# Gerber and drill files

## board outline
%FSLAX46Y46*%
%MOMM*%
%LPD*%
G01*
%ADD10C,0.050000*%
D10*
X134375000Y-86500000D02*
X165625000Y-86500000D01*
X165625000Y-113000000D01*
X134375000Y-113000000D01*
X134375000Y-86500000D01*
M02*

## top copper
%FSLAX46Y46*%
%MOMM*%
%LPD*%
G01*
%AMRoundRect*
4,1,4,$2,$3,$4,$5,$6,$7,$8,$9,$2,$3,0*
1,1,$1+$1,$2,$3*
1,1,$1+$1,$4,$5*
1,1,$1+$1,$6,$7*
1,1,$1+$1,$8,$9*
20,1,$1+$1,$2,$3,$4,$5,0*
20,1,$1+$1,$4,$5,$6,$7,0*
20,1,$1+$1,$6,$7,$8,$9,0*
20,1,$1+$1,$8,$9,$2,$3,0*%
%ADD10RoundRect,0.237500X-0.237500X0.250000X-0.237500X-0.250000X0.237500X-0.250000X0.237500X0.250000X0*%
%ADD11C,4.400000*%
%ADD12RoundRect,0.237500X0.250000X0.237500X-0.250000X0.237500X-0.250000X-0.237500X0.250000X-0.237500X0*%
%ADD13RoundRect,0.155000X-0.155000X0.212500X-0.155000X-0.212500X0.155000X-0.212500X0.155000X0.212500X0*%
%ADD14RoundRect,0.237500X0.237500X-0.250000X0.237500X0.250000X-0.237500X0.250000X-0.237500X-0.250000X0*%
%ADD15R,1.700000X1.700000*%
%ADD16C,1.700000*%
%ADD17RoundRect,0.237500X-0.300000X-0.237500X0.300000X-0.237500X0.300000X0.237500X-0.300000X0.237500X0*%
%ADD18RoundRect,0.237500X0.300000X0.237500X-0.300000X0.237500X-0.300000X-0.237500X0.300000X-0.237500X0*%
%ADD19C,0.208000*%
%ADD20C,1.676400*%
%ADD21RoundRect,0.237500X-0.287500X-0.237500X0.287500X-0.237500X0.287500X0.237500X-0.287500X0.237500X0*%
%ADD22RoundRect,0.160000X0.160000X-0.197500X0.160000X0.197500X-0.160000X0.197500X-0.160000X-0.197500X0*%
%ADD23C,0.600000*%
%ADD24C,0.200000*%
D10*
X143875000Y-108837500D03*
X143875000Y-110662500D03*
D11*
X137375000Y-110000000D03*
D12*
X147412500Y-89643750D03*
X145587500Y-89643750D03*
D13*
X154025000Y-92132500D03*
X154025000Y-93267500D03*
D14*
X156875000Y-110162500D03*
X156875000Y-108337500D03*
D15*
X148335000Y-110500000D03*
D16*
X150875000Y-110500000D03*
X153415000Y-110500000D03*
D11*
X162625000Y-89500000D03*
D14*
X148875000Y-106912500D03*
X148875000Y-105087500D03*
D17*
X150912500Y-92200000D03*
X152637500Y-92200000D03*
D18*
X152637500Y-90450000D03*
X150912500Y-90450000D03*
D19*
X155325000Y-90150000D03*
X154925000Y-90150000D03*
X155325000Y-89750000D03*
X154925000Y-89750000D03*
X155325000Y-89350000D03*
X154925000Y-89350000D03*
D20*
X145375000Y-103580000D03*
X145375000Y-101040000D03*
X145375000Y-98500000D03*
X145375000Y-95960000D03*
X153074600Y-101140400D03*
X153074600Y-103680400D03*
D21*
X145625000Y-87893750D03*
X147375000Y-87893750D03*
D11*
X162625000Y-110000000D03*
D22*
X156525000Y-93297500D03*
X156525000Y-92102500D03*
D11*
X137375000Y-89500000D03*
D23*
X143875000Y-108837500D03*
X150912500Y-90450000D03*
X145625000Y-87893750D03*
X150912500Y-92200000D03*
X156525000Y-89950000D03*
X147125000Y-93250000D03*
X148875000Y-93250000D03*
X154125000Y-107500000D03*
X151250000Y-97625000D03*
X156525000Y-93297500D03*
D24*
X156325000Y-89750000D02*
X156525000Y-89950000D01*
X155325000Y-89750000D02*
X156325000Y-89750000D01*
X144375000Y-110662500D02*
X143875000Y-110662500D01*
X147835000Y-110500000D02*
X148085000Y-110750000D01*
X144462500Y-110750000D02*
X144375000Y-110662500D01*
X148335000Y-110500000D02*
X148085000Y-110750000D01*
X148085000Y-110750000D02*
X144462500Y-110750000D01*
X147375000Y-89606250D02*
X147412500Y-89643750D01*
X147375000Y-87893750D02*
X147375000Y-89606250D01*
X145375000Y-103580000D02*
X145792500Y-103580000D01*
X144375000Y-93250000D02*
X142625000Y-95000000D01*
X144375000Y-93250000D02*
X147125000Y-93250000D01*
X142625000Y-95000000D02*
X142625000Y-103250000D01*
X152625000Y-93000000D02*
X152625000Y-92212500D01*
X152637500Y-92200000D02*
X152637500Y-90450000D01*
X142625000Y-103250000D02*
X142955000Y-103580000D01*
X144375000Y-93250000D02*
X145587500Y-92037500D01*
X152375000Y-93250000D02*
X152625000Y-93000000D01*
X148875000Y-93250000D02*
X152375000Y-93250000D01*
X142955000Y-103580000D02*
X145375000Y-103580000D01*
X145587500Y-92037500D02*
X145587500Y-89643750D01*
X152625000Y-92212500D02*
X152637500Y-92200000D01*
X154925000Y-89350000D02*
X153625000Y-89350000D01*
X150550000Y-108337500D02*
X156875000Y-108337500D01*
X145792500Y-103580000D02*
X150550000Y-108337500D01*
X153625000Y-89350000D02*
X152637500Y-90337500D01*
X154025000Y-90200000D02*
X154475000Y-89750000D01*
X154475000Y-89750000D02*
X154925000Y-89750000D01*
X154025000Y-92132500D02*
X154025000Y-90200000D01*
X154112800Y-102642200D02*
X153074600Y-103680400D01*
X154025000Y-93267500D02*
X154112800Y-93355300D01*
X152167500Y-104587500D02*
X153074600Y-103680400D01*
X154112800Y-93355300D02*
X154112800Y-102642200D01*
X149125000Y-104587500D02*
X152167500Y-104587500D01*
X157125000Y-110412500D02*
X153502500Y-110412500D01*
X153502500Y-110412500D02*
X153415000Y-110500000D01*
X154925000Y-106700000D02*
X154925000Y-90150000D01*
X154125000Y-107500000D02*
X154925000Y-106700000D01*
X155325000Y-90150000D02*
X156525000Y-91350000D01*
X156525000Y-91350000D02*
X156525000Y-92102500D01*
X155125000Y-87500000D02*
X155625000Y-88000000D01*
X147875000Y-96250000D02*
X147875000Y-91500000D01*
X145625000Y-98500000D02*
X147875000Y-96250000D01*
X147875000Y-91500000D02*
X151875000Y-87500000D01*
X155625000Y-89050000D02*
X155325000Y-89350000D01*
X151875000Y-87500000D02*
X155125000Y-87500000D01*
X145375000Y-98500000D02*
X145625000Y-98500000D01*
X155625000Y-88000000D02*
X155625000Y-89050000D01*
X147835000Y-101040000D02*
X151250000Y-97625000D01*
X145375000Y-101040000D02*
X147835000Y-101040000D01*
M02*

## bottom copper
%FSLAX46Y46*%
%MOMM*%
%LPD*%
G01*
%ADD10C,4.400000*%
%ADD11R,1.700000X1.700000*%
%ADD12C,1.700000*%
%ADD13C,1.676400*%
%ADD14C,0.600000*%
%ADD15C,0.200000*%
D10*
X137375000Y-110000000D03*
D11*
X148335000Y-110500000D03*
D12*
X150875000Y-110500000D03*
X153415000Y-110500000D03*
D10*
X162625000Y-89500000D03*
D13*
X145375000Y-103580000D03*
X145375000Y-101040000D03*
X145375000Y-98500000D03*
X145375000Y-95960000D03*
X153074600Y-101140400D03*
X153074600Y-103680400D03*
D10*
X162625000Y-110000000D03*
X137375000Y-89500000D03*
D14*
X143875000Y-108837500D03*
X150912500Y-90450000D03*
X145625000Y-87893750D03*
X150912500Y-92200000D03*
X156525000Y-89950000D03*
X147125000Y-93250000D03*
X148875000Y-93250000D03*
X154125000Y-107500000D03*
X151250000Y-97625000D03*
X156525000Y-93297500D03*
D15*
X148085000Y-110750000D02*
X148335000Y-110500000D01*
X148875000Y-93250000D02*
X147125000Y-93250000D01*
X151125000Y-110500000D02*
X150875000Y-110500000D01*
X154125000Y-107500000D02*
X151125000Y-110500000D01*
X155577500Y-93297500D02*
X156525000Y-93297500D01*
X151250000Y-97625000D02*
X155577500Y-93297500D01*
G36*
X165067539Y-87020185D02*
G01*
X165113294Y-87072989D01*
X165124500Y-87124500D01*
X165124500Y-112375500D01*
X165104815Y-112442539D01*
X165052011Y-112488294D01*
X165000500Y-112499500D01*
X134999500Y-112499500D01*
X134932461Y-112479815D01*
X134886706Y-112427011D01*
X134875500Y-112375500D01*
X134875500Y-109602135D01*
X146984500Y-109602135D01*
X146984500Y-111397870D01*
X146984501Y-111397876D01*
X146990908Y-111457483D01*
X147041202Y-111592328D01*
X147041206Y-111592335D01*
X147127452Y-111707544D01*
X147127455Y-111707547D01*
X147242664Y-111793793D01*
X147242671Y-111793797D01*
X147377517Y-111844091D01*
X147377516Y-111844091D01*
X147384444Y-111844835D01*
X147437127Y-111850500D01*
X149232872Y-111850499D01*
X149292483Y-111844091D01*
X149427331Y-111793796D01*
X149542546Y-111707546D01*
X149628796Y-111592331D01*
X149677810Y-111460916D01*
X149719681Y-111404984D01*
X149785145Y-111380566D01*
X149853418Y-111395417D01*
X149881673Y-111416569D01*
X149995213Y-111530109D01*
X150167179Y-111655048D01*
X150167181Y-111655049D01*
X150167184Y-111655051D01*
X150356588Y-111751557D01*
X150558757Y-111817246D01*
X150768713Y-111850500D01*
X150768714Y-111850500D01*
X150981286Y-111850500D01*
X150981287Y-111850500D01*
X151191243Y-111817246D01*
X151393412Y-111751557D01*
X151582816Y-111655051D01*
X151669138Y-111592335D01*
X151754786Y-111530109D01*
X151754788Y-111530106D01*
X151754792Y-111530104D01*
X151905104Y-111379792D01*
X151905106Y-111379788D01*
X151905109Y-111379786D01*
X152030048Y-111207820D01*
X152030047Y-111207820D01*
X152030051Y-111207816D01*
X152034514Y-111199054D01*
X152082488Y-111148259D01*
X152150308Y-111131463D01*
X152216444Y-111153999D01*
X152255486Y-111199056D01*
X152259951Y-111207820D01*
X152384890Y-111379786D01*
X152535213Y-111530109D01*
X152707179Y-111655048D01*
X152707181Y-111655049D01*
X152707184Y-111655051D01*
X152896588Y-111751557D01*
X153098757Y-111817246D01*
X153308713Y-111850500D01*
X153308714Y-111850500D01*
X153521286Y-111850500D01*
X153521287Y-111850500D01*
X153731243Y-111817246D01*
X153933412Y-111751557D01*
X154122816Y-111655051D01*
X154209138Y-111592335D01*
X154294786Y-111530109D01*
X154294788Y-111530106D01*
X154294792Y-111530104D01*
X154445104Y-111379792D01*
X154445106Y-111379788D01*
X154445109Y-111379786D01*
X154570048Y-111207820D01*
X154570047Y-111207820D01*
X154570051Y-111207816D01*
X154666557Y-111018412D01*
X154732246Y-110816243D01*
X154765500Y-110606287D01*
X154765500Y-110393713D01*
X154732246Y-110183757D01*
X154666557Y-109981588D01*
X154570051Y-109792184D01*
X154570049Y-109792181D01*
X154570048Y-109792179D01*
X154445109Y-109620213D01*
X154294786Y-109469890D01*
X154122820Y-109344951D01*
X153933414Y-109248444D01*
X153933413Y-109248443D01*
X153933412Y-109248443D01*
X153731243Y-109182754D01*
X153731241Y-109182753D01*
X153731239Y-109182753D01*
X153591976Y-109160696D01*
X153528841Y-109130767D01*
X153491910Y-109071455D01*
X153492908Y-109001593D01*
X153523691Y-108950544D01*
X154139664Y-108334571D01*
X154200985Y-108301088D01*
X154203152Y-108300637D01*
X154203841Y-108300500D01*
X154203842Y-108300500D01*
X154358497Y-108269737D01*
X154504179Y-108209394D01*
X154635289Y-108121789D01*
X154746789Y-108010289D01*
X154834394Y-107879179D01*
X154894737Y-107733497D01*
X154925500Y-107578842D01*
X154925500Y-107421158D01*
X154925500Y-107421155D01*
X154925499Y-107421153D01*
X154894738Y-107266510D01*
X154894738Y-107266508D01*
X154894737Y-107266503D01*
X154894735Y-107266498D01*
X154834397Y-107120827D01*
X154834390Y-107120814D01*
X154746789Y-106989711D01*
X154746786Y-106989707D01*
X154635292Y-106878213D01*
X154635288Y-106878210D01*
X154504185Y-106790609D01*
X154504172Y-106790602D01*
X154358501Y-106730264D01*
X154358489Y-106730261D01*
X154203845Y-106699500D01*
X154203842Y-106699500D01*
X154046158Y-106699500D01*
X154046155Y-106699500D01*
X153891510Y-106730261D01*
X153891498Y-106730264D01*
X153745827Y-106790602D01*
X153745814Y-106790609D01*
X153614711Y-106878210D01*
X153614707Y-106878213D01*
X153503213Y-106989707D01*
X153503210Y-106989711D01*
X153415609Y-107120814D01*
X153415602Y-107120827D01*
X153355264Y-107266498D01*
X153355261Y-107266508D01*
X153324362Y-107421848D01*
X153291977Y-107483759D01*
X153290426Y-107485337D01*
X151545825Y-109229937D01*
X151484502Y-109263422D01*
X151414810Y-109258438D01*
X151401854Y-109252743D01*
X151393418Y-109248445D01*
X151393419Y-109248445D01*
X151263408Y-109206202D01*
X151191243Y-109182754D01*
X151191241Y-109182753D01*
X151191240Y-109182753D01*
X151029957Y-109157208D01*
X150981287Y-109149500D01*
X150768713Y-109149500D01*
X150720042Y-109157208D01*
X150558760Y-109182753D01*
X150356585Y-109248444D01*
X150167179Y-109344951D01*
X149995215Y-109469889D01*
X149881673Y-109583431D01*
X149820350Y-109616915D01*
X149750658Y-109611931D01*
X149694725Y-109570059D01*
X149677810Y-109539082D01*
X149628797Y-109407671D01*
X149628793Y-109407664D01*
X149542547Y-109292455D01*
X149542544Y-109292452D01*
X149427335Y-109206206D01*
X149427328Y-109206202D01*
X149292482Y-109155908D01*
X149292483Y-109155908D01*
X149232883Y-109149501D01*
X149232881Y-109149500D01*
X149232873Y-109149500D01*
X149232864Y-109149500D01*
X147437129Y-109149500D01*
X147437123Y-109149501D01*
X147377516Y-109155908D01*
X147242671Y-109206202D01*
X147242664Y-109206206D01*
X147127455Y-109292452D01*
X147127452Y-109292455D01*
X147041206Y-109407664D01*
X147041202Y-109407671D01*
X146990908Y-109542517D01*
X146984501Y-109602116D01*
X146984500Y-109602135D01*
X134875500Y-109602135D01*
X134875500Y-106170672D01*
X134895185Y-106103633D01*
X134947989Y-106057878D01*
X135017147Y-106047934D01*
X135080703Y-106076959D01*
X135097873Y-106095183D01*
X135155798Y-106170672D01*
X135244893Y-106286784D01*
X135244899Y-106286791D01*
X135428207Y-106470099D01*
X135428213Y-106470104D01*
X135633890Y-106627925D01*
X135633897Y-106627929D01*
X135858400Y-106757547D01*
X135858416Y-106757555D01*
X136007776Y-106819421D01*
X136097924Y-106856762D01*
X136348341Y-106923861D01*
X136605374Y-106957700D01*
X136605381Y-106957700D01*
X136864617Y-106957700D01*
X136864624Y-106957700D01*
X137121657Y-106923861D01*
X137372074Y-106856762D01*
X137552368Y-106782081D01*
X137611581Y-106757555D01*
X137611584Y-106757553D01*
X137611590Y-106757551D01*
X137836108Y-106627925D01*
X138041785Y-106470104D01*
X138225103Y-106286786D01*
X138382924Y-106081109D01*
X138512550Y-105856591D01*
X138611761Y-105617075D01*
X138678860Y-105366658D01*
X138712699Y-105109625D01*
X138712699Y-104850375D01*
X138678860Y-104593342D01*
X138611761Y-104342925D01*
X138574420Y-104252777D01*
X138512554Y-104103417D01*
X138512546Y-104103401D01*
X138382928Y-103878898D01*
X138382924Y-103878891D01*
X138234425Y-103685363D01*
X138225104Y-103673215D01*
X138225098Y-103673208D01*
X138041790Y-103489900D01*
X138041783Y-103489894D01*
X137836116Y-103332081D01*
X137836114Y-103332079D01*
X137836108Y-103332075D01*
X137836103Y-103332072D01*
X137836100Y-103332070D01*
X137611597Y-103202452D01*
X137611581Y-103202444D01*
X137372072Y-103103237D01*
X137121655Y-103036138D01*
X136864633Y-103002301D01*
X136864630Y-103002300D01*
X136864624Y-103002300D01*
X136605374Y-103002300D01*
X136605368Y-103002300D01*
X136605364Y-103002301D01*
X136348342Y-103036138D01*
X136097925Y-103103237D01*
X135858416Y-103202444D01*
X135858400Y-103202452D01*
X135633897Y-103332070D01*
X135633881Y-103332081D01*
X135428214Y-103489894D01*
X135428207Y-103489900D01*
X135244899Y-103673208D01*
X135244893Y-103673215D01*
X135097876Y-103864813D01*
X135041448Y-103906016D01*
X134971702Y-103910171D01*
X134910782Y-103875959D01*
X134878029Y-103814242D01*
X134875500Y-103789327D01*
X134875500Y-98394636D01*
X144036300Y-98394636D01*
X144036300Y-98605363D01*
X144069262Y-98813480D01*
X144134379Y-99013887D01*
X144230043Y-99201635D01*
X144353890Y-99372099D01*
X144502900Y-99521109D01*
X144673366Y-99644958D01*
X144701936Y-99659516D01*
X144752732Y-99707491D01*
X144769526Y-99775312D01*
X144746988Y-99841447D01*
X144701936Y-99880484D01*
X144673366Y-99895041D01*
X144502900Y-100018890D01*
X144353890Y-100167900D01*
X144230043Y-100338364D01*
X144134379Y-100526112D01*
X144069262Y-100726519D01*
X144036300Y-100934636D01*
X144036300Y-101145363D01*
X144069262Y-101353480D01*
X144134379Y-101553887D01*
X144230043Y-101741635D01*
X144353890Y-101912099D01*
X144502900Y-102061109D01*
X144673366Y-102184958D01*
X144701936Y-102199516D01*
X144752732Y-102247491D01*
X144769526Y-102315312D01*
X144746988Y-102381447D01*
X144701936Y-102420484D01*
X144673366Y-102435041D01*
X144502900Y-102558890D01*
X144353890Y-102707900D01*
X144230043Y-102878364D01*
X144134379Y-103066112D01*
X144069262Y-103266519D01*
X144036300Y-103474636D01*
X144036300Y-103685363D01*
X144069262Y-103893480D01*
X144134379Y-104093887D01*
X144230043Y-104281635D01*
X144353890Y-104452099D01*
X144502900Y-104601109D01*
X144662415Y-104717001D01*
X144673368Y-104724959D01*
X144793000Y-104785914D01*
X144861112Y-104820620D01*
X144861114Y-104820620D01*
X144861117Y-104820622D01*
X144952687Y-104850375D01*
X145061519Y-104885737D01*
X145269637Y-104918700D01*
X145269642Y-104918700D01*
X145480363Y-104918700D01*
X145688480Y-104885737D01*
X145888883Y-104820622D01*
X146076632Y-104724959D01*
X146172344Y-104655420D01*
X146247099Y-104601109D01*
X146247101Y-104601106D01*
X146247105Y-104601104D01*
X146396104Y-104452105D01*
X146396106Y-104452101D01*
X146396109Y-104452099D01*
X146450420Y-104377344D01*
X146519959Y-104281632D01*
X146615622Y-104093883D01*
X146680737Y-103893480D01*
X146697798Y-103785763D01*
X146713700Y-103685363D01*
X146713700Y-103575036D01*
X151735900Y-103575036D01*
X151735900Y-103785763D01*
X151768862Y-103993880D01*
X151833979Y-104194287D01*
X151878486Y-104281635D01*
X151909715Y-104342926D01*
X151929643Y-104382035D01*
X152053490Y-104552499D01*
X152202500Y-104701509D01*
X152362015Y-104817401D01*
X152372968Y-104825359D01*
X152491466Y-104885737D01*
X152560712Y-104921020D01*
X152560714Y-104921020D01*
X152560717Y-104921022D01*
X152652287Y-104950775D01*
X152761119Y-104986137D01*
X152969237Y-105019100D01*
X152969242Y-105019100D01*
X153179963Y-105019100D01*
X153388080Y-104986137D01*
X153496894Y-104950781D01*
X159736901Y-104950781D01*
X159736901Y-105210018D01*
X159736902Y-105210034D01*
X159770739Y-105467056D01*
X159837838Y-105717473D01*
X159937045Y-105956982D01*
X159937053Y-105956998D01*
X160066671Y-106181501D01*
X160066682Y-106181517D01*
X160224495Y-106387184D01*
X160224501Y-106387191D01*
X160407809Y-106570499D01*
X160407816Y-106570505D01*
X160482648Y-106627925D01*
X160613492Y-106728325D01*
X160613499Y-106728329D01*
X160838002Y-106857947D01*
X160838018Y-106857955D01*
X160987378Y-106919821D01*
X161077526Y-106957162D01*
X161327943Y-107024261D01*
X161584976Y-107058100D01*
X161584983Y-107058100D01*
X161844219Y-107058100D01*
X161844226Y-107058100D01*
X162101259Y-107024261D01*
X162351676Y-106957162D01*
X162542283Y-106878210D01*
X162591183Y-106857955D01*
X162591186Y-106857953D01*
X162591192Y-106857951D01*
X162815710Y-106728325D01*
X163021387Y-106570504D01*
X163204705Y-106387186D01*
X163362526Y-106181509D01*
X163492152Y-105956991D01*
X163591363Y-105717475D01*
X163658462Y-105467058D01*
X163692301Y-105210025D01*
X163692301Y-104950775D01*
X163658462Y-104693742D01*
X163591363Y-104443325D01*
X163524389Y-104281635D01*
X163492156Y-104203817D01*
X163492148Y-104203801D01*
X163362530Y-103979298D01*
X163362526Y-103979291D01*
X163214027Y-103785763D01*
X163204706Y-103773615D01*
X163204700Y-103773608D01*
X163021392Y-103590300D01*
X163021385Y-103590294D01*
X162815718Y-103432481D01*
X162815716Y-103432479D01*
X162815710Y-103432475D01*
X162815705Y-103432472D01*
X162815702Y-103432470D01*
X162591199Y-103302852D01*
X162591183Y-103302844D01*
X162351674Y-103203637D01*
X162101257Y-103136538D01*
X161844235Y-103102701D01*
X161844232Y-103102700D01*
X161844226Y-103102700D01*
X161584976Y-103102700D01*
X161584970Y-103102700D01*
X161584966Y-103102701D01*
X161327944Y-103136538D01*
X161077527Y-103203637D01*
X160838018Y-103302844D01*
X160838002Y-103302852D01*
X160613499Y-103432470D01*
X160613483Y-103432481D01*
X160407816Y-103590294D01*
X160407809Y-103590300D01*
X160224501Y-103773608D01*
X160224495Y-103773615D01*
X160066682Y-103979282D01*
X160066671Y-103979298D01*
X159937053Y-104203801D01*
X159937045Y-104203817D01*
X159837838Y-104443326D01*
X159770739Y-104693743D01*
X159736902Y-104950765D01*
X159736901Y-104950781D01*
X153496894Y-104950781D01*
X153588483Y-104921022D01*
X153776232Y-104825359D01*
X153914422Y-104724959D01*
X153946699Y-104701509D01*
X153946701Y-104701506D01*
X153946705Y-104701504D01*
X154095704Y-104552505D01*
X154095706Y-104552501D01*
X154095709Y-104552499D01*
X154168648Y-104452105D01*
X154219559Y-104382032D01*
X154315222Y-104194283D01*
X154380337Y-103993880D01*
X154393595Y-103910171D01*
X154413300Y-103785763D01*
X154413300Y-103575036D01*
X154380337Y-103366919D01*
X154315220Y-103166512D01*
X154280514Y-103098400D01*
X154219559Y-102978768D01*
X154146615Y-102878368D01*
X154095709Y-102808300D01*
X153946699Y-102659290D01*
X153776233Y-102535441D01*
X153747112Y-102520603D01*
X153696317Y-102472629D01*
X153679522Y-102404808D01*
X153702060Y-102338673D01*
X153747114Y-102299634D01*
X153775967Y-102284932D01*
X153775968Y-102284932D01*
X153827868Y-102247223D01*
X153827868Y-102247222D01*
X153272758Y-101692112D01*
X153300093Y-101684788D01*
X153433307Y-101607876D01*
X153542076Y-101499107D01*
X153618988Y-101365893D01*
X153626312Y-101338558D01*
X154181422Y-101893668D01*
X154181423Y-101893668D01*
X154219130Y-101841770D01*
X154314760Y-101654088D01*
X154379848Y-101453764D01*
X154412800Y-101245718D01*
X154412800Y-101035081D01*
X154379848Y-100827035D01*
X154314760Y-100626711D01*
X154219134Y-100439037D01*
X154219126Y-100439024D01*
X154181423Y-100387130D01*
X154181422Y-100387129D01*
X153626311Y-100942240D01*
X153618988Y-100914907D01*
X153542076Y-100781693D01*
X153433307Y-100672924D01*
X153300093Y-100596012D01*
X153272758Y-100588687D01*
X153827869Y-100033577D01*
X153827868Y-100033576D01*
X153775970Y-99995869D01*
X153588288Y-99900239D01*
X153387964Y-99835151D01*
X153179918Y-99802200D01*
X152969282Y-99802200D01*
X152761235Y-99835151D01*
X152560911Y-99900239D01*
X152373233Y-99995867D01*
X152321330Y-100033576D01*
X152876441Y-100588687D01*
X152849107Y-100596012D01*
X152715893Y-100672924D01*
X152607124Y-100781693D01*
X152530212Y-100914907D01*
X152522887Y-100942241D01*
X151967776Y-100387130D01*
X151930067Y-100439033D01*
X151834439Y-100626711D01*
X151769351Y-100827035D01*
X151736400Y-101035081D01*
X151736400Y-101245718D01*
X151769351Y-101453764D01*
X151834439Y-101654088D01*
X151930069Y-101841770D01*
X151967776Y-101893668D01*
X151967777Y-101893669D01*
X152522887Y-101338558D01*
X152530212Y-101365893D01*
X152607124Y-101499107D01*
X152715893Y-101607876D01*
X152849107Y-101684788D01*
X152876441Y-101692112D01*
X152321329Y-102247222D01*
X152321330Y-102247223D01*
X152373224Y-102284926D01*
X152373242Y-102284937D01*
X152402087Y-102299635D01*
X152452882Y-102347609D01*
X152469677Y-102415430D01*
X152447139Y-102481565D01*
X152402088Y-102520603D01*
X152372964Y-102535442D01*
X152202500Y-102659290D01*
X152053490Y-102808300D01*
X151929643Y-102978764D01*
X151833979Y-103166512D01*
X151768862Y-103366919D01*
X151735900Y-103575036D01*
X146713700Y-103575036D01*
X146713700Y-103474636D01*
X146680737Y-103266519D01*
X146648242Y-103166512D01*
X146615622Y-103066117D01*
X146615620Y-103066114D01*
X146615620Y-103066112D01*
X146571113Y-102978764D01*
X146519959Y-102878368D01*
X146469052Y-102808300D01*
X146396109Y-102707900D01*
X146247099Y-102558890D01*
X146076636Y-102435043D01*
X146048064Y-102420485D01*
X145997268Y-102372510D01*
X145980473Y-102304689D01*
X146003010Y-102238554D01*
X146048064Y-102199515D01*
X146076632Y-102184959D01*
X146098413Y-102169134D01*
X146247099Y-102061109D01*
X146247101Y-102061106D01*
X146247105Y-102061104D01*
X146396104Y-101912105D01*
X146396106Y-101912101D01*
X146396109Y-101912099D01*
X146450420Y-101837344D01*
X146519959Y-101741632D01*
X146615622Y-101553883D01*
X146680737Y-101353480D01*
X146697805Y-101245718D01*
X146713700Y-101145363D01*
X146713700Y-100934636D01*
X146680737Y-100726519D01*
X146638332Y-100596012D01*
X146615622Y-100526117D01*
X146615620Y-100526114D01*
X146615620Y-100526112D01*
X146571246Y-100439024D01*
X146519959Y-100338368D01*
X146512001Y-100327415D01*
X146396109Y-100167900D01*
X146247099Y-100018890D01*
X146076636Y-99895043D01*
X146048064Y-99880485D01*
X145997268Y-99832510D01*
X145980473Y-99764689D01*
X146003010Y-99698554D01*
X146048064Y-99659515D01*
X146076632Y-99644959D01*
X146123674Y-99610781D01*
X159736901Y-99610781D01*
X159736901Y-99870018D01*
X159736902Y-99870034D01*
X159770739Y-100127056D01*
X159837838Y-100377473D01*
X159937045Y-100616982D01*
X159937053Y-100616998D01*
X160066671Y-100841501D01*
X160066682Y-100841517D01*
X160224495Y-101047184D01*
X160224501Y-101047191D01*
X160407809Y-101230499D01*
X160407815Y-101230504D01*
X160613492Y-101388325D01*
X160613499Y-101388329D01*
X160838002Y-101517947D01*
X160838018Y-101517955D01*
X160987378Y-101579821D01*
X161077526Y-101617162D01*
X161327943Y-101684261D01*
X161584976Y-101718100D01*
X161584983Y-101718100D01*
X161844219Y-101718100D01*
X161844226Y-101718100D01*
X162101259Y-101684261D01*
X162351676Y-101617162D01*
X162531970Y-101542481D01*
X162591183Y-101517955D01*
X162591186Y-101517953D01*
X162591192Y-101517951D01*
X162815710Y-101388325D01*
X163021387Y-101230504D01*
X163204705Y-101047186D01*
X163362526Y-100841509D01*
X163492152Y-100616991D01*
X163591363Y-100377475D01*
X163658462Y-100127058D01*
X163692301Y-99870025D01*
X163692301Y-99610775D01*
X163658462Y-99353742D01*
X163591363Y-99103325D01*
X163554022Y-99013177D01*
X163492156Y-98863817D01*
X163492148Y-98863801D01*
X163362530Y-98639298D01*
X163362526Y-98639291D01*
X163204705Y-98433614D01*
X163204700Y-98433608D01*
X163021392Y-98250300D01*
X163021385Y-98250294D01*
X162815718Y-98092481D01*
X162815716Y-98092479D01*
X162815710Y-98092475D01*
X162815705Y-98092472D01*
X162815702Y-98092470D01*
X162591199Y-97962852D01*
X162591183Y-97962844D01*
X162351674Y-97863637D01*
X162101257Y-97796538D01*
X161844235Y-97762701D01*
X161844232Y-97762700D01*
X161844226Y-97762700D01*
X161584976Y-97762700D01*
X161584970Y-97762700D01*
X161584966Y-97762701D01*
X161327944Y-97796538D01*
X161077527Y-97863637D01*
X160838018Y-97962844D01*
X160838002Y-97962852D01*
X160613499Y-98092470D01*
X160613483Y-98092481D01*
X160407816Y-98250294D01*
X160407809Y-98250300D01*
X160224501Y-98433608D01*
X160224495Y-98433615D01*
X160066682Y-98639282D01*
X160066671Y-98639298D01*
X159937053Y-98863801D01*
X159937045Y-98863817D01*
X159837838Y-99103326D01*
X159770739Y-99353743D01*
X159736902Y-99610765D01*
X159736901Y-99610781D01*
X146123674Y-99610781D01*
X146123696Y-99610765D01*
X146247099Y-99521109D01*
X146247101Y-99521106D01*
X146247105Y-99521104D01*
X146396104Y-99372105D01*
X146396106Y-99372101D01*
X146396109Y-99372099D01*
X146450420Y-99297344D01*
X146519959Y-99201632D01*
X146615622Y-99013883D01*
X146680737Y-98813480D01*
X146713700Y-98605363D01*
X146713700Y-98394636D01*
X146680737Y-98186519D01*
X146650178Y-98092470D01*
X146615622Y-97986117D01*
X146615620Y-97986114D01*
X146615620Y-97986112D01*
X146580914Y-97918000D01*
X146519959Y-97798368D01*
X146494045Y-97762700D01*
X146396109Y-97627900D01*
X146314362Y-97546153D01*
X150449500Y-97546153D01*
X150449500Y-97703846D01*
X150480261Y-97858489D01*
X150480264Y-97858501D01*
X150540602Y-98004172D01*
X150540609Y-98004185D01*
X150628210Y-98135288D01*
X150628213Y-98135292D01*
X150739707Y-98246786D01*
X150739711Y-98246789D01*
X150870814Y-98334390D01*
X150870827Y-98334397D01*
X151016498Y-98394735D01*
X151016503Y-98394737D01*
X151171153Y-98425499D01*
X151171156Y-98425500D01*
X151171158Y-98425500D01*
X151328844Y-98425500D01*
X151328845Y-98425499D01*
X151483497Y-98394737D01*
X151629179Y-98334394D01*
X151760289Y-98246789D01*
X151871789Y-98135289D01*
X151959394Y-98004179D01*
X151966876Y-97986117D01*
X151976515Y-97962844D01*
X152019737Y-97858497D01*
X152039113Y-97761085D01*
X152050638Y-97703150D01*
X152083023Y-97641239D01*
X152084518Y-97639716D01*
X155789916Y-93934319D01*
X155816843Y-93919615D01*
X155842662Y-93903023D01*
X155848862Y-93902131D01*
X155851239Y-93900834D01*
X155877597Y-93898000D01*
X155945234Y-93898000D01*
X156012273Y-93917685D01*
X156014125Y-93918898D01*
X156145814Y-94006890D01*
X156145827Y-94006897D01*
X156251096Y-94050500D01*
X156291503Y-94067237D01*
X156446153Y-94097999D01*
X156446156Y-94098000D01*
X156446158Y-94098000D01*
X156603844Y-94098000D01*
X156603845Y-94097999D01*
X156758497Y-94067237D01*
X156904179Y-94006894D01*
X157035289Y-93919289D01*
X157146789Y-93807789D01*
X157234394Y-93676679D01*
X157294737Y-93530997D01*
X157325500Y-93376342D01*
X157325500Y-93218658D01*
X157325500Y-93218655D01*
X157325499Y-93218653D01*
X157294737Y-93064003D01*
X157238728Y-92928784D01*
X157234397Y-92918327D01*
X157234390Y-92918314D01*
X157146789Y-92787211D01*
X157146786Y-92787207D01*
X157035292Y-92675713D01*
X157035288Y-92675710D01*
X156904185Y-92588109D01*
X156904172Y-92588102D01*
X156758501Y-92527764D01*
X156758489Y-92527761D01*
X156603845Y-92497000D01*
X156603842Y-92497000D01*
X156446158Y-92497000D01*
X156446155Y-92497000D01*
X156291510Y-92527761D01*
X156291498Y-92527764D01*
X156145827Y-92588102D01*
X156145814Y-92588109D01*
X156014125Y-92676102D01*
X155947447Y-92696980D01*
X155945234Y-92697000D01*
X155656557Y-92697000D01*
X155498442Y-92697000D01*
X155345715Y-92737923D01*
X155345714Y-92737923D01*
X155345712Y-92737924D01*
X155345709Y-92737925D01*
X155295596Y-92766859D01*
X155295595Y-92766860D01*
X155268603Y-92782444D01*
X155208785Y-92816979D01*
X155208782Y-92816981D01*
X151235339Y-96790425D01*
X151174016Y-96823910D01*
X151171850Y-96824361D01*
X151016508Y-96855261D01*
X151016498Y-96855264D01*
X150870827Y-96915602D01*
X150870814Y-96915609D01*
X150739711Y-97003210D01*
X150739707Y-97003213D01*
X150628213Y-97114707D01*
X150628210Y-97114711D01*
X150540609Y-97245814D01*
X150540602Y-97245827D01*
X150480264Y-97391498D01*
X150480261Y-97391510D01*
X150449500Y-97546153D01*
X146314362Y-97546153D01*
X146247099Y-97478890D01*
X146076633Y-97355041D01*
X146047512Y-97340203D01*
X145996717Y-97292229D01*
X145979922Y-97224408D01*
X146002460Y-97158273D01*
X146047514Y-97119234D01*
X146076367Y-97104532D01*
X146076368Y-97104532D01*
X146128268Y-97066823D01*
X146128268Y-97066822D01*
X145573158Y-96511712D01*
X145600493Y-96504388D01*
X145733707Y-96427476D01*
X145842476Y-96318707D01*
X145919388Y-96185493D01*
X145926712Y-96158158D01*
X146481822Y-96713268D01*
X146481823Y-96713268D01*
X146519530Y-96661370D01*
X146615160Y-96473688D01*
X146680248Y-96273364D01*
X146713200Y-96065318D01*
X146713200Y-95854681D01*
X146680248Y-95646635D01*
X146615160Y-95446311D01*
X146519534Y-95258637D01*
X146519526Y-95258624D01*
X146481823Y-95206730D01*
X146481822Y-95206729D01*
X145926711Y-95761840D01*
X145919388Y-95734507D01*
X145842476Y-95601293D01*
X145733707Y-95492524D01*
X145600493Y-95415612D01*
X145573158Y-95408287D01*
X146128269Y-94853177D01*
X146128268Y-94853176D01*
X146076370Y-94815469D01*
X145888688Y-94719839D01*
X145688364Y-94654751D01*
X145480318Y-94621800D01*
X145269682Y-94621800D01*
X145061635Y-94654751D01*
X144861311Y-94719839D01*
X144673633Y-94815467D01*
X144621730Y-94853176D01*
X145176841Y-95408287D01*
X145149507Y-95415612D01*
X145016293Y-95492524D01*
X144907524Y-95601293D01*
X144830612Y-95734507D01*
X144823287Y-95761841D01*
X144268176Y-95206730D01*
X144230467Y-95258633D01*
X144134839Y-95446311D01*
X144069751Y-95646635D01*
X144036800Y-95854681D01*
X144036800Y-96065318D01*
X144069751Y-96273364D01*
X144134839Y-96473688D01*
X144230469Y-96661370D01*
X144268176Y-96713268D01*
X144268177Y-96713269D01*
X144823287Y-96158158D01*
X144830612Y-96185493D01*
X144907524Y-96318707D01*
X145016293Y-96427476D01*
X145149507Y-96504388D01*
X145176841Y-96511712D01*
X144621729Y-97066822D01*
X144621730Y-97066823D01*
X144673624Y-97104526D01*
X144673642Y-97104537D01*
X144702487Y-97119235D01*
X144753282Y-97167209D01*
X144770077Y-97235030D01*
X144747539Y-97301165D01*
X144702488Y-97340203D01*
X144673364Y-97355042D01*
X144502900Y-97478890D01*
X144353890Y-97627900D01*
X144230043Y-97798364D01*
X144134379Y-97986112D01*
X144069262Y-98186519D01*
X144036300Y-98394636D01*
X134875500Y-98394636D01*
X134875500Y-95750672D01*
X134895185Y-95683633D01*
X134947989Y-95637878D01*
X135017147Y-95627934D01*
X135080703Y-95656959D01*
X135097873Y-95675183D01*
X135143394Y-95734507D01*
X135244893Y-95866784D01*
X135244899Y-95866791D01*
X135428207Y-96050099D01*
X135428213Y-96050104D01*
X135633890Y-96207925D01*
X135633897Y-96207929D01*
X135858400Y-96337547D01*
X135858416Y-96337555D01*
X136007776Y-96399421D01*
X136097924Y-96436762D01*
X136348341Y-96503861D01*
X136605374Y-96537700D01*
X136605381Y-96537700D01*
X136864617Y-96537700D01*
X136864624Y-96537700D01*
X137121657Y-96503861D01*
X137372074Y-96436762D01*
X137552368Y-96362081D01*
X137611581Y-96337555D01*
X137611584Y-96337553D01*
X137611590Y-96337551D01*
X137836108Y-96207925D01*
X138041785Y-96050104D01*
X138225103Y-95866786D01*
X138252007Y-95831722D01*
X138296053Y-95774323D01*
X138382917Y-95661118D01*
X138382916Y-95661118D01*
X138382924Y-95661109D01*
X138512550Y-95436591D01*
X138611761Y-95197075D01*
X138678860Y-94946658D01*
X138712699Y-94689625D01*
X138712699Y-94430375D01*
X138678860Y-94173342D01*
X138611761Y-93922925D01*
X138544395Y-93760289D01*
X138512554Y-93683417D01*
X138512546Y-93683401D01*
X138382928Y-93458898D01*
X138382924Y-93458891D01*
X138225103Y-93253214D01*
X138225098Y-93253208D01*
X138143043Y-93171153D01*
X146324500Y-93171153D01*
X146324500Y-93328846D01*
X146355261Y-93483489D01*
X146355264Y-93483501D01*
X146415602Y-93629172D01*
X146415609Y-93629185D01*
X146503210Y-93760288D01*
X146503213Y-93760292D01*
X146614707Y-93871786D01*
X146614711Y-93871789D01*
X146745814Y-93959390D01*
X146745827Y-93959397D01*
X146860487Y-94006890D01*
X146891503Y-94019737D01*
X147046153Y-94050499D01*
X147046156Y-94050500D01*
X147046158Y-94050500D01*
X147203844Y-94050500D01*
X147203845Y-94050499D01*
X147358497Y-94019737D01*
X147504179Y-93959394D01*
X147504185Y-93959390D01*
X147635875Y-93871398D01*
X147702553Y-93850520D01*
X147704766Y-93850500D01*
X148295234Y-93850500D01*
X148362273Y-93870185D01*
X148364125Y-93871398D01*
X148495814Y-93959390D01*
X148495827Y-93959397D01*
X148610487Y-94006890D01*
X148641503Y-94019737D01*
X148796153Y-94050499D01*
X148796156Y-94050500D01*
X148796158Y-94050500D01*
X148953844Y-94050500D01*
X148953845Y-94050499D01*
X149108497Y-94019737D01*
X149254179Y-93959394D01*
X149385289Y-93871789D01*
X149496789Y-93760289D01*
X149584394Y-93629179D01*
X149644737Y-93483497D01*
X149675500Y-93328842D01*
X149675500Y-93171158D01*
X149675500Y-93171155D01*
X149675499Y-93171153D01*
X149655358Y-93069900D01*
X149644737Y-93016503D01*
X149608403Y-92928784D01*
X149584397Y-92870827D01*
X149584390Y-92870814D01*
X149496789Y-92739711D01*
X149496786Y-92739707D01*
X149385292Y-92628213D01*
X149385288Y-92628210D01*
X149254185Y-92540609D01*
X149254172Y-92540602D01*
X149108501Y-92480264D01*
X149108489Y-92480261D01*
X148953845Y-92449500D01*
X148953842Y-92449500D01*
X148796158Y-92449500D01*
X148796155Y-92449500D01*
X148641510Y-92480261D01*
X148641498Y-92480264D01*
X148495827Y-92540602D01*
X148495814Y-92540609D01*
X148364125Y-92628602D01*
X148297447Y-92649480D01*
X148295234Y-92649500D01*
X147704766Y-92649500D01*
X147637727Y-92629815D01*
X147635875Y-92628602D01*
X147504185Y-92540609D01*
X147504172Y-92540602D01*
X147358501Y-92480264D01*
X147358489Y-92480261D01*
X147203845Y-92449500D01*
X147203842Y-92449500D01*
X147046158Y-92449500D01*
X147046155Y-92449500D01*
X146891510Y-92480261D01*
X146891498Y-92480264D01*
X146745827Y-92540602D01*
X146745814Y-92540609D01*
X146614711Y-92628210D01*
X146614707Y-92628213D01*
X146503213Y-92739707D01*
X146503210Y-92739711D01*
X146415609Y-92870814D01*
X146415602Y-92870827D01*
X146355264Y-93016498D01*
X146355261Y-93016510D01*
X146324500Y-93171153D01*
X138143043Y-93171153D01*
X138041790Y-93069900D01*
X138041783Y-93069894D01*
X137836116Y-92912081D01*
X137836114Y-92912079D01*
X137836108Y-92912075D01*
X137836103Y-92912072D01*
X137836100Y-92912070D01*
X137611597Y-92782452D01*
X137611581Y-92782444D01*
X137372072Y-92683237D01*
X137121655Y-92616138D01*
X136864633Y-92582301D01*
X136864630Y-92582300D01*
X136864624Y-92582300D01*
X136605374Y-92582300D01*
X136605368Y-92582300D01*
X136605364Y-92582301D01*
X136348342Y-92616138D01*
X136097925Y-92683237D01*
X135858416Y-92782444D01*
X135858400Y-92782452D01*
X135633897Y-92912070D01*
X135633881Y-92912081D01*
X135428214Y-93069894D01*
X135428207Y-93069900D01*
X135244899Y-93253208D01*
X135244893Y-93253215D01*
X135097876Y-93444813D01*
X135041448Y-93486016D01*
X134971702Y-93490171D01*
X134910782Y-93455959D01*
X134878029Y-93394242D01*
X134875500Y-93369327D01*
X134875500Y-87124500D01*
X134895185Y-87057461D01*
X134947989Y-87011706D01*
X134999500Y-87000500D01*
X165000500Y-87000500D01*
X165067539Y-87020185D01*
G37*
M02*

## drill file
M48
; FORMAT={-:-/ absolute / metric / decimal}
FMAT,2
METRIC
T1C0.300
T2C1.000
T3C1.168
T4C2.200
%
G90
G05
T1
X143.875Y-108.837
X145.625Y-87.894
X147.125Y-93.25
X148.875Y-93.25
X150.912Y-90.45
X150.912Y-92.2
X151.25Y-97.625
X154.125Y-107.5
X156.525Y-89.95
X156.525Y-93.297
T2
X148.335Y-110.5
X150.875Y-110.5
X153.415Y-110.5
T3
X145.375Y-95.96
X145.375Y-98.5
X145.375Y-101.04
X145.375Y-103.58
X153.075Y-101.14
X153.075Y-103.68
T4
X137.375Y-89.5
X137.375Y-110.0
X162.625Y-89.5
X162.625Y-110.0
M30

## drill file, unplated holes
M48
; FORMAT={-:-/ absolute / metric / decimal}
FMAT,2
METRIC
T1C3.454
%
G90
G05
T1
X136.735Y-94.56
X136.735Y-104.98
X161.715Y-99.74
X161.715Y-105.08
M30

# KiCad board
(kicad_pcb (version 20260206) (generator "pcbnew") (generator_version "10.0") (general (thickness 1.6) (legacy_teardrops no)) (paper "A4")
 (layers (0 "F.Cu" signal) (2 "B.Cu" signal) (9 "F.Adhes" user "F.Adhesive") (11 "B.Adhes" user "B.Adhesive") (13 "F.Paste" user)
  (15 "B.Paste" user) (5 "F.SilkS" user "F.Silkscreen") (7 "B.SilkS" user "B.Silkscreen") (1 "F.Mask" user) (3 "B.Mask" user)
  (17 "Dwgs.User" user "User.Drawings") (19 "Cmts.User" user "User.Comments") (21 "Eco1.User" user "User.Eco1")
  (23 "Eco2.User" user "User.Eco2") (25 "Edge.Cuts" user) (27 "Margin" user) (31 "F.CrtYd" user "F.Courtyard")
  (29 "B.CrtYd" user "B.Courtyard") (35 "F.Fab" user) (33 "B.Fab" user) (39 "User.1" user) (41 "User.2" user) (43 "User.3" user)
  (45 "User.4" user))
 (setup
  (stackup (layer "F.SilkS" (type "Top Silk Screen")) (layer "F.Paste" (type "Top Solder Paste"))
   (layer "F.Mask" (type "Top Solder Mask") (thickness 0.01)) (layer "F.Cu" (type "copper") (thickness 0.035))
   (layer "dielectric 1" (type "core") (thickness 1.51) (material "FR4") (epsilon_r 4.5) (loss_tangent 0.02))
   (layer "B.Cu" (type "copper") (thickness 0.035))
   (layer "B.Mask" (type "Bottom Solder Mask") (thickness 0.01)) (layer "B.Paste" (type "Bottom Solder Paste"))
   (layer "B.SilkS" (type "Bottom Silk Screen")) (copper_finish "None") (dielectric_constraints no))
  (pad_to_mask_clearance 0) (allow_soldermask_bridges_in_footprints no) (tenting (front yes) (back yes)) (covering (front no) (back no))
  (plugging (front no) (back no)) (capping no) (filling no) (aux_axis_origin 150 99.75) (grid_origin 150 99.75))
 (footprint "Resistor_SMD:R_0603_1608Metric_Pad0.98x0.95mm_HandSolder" (layer "F.Cu") (at 143.875 109.75 -90)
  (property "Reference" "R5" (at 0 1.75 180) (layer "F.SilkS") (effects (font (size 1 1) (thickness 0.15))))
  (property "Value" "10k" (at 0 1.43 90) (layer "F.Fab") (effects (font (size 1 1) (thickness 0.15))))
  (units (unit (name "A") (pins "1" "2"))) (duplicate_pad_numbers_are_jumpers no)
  (pad "1" smd roundrect (at -0.9125 0 270) (size 0.975 0.95) (layers "F.Cu" "F.Mask" "F.Paste") (roundrect_rratio 0.25) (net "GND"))
  (pad "2" smd roundrect (at 0.9125 0 270) (size 0.975 0.95) (layers "F.Cu" "F.Mask" "F.Paste") (roundrect_rratio 0.25) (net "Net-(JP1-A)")))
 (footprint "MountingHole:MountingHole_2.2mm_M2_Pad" (layer "F.Cu") (at 137.375 110)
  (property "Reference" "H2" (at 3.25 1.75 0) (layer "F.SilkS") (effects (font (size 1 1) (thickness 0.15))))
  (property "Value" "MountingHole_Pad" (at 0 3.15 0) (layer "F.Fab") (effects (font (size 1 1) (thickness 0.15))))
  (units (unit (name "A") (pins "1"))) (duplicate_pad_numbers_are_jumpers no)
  (pad "1" thru_hole circle (at 0 0) (size 4.4 4.4) (drill 2.2) (layers "*.Cu" "*.Mask") (remove_unused_layers no) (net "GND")
   (zone_connect 2)))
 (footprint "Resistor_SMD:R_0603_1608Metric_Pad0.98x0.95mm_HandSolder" (layer "F.Cu") (at 146.5 89.64375 180)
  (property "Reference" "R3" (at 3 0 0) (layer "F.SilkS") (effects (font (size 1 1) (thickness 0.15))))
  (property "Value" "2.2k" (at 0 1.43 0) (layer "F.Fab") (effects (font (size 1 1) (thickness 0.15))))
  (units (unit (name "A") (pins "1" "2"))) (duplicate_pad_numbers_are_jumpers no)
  (pad "1" smd roundrect (at -0.9125 0 180) (size 0.975 0.95) (layers "F.Cu" "F.Mask" "F.Paste") (roundrect_rratio 0.25) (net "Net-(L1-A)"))
  (pad "2" smd roundrect (at 0.9125 0 180) (size 0.975 0.95) (layers "F.Cu" "F.Mask" "F.Paste") (roundrect_rratio 0.25) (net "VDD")))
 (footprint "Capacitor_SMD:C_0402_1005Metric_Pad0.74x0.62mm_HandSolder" (layer "F.Cu") (at 154.025 92.7 -90)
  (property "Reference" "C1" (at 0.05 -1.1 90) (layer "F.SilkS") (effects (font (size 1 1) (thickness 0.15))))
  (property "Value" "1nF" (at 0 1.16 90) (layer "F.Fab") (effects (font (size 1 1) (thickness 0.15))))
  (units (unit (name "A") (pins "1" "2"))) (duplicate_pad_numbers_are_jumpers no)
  (pad "1" smd roundrect (at -0.5675 0 270) (size 0.735 0.62) (layers "F.Cu" "F.Mask" "F.Paste") (roundrect_rratio 0.25)
   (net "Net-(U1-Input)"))
  (pad "2" smd roundrect (at 0.5675 0 270) (size 0.735 0.62) (layers "F.Cu" "F.Mask" "F.Paste") (roundrect_rratio 0.25) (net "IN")))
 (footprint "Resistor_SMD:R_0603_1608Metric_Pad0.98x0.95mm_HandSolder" (layer "F.Cu") (at 156.875 109.25 90)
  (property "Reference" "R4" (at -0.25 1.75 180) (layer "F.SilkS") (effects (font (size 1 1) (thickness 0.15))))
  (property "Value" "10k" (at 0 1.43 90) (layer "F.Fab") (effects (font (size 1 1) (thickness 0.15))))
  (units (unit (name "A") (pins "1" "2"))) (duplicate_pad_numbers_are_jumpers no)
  (pad "1" smd roundrect (at -0.9125 0 90) (size 0.975 0.95) (layers "F.Cu" "F.Mask" "F.Paste") (roundrect_rratio 0.25) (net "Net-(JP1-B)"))
  (pad "2" smd roundrect (at 0.9125 0 90) (size 0.975 0.95) (layers "F.Cu" "F.Mask" "F.Paste") (roundrect_rratio 0.25) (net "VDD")))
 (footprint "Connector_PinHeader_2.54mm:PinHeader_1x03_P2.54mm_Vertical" (layer "F.Cu") (at 148.335 110.5 90)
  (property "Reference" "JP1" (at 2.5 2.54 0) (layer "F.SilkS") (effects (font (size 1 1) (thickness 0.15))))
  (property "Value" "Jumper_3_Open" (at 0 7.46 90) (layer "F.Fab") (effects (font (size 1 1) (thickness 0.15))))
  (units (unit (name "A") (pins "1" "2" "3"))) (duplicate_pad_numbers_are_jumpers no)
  (pad "1" thru_hole rect (at 0 0 90) (size 1.7 1.7) (drill 1) (layers "*.Cu" "*.Mask") (remove_unused_layers no) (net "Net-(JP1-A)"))
  (pad "2" thru_hole circle (at 0 2.54 90) (size 1.7 1.7) (drill 1) (layers "*.Cu" "*.Mask") (remove_unused_layers no) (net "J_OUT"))
  (pad "3" thru_hole circle (at 0 5.08 90) (size 1.7 1.7) (drill 1) (layers "*.Cu" "*.Mask") (remove_unused_layers no) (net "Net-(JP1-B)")))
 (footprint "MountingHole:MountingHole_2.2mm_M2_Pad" (layer "F.Cu") (at 162.625 89.5)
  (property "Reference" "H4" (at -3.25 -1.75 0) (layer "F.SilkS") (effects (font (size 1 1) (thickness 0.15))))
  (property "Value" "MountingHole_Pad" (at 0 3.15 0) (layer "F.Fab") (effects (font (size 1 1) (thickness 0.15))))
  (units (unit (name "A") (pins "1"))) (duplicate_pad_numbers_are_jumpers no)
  (pad "1" thru_hole circle (at 0 0) (size 4.4 4.4) (drill 2.2) (layers "*.Cu" "*.Mask") (remove_unused_layers no) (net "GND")
   (zone_connect 2)))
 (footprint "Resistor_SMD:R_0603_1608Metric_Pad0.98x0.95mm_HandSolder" (layer "F.Cu") (at 148.875 106 90)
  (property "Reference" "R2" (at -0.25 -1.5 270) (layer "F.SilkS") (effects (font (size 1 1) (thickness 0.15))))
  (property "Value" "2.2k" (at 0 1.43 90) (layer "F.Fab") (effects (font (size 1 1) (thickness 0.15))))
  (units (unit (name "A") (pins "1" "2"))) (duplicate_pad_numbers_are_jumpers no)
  (pad "1" smd roundrect (at -0.9125 0 90) (size 0.975 0.95) (layers "F.Cu" "F.Mask" "F.Paste") (roundrect_rratio 0.25) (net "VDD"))
  (pad "2" smd roundrect (at 0.9125 0 90) (size 0.975 0.95) (layers "F.Cu" "F.Mask" "F.Paste") (roundrect_rratio 0.25) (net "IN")))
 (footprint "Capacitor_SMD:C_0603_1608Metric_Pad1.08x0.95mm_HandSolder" (layer "F.Cu") (at 151.775 92.2)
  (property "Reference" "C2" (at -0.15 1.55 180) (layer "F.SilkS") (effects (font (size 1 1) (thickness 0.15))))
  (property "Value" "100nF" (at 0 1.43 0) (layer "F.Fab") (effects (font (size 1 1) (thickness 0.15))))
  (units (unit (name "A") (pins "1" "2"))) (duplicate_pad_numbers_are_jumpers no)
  (pad "1" smd roundrect (at -0.8625 0) (size 1.075 0.95) (layers "F.Cu" "F.Mask" "F.Paste") (roundrect_rratio 0.25) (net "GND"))
  (pad "2" smd roundrect (at 0.8625 0) (size 1.075 0.95) (layers "F.Cu" "F.Mask" "F.Paste") (roundrect_rratio 0.25) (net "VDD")))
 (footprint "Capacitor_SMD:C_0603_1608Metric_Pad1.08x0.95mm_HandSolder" (layer "F.Cu") (at 151.775 90.45 180)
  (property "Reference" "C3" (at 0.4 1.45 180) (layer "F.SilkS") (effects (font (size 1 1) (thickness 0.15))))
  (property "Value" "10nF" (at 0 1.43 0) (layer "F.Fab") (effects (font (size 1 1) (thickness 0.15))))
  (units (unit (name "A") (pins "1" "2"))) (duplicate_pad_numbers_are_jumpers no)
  (pad "1" smd roundrect (at -0.8625 0 180) (size 1.075 0.95) (layers "F.Cu" "F.Mask" "F.Paste") (roundrect_rratio 0.25) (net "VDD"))
  (pad "2" smd roundrect (at 0.8625 0 180) (size 1.075 0.95) (layers "F.Cu" "F.Mask" "F.Paste") (roundrect_rratio 0.25) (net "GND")))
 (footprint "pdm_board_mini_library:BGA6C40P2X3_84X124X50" (layer "F.Cu") (at 155.125 89.75 180)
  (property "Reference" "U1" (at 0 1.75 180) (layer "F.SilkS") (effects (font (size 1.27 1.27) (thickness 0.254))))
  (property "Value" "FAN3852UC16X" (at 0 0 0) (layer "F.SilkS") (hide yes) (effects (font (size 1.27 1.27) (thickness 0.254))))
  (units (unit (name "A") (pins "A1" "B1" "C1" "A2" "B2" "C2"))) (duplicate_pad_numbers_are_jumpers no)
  (pad "A1" smd circle (at -0.2 -0.4 270) (size 0.208 0.208) (layers "F.Cu" "F.Mask" "F.Paste") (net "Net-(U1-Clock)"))
  (pad "A2" smd circle (at 0.2 -0.4 270) (size 0.208 0.208) (layers "F.Cu" "F.Mask" "F.Paste") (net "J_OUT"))
  (pad "B1" smd circle (at -0.2 0 270) (size 0.208 0.208) (layers "F.Cu" "F.Mask" "F.Paste") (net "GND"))
  (pad "B2" smd circle (at 0.2 0 270) (size 0.208 0.208) (layers "F.Cu" "F.Mask" "F.Paste") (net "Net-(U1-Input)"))
  (pad "C1" smd circle (at -0.2 0.4 270) (size 0.208 0.208) (layers "F.Cu" "F.Mask" "F.Paste") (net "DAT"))
  (pad "C2" smd circle (at 0.2 0.4 270) (size 0.208 0.208) (layers "F.Cu" "F.Mask" "F.Paste") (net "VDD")))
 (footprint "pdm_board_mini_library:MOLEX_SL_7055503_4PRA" (layer "F.Cu") (at 145.375 103.58 -90)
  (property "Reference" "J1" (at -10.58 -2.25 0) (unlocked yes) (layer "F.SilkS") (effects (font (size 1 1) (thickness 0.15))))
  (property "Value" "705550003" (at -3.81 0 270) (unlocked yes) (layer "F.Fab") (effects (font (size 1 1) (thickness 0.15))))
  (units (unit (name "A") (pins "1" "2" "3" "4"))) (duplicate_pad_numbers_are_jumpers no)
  (pad "" np_thru_hole circle (at -9.02 8.640001 270) (size 3.4544 3.4544) (drill 3.4544) (layers))
  (pad "" np_thru_hole circle (at 1.4 8.640001 270) (size 3.4544 3.4544) (drill 3.4544) (layers))
  (pad "1" thru_hole circle (at 0 0 270) (size 1.6764 1.6764) (drill 1.1684) (layers "*.Cu" "*.Mask") (remove_unused_layers no) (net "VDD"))
  (pad "2" thru_hole circle (at -2.54 0 270) (size 1.6764 1.6764) (drill 1.1684) (layers "*.Cu" "*.Mask") (remove_unused_layers no)
   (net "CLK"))
  (pad "3" thru_hole circle (at -5.08 0 270) (size 1.6764 1.6764) (drill 1.1684) (layers "*.Cu" "*.Mask") (remove_unused_layers no)
   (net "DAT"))
  (pad "4" thru_hole circle (at -7.62 0 270) (size 1.6764 1.6764) (drill 1.1684) (layers "*.Cu" "*.Mask") (remove_unused_layers no)
   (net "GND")))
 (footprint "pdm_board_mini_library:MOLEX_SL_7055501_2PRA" (layer "F.Cu") (at 153.0746 101.1404 90)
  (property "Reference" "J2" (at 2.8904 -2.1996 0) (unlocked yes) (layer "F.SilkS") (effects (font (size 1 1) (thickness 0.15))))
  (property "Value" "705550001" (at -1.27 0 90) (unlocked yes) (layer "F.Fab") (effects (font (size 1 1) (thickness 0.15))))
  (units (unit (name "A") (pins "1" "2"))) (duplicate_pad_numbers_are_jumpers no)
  (pad "" np_thru_hole circle (at -3.94 8.640001 90) (size 3.4544 3.4544) (drill 3.4544) (layers))
  (pad "" np_thru_hole circle (at 1.4 8.640001 90) (size 3.4544 3.4544) (drill 3.4544) (layers))
  (pad "1" thru_hole circle (at 0 0 90) (size 1.6764 1.6764) (drill 1.1684) (layers "*.Cu" "*.Mask") (remove_unused_layers no) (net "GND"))
  (pad "2" thru_hole circle (at -2.54 0 90) (size 1.6764 1.6764) (drill 1.1684) (layers "*.Cu" "*.Mask") (remove_unused_layers no)
   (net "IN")))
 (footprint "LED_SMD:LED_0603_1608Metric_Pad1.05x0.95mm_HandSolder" (layer "F.Cu") (at 146.5 87.89375)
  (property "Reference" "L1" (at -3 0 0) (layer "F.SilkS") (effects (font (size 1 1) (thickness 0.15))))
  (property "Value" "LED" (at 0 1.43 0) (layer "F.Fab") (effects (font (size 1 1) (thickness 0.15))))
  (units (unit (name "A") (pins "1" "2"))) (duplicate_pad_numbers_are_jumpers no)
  (pad "1" smd roundrect (at -0.875 0) (size 1.05 0.95) (layers "F.Cu" "F.Mask" "F.Paste") (roundrect_rratio 0.25) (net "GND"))
  (pad "2" smd roundrect (at 0.875 0) (size 1.05 0.95) (layers "F.Cu" "F.Mask" "F.Paste") (roundrect_rratio 0.25) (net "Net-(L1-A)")))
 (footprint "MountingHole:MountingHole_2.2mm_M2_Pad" (layer "F.Cu") (at 162.625 110)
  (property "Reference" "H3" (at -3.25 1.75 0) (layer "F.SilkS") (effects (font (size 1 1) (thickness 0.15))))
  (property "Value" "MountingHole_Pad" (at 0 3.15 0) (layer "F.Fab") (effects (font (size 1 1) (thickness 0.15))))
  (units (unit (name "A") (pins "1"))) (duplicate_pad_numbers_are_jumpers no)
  (pad "1" thru_hole circle (at 0 0) (size 4.4 4.4) (drill 2.2) (layers "*.Cu" "*.Mask") (remove_unused_layers no) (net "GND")
   (zone_connect 2)))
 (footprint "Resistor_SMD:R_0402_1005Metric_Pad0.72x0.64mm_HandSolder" (layer "F.Cu") (at 156.525 92.7 90)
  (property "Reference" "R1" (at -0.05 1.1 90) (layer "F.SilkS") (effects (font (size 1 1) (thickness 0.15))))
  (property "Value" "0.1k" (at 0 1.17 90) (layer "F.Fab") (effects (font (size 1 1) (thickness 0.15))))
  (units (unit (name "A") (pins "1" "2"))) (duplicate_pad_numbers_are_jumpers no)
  (pad "1" smd roundrect (at -0.5975 0 90) (size 0.715 0.64) (layers "F.Cu" "F.Mask" "F.Paste") (roundrect_rratio 0.25) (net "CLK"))
  (pad "2" smd roundrect (at 0.5975 0 90) (size 0.715 0.64) (layers "F.Cu" "F.Mask" "F.Paste") (roundrect_rratio 0.25)
   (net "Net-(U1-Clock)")))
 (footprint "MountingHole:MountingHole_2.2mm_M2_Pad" (layer "F.Cu") (at 137.375 89.5)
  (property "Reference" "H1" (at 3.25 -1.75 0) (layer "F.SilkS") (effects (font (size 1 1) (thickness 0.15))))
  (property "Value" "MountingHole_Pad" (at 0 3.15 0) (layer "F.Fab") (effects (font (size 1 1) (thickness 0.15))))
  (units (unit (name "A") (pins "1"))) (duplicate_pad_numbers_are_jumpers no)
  (pad "1" thru_hole circle (at 0 0) (size 4.4 4.4) (drill 2.2) (layers "*.Cu" "*.Mask") (remove_unused_layers no) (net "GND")
   (zone_connect 2)))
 (gr_rect (start 134.375 86.5) (end 165.625 113) (stroke (width 0.05) (type default)) (fill no) (layer "Edge.Cuts"))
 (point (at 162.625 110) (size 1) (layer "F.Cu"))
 (segment (start 156.325 89.75) (end 156.525 89.95) (width 0.2) (layer "F.Cu") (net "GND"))
 (segment (start 155.325 89.75) (end 156.325 89.75) (width 0.2) (layer "F.Cu") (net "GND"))
 (via (at 143.875 108.8375) (size 0.6) (drill 0.3) (layers "F.Cu" "B.Cu") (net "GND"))
 (via (at 150.9125 90.45) (size 0.6) (drill 0.3) (layers "F.Cu" "B.Cu") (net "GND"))
 (via (at 145.625 87.89375) (size 0.6) (drill 0.3) (layers "F.Cu" "B.Cu") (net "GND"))
 (via (at 150.9125 92.2) (size 0.6) (drill 0.3) (layers "F.Cu" "B.Cu") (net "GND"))
 (via (at 156.525 89.95) (size 0.6) (drill 0.3) (layers "F.Cu" "B.Cu") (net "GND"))
 (segment (start 144.375 110.6625) (end 143.875 110.6625) (width 0.2) (layer "F.Cu") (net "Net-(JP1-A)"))
 (segment (start 147.835 110.5) (end 148.085 110.75) (width 0.2) (layer "F.Cu") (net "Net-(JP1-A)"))
 (segment (start 144.4625 110.75) (end 144.375 110.6625) (width 0.2) (layer "F.Cu") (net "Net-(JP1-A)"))
 (segment (start 148.335 110.5) (end 148.085 110.75) (width 0.2) (layer "F.Cu") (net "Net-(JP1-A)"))
 (segment (start 148.085 110.75) (end 144.4625 110.75) (width 0.2) (layer "F.Cu") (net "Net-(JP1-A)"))
 (segment (start 148.085 110.75) (end 148.335 110.5) (width 0.2) (layer "B.Cu") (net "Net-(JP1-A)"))
 (segment (start 147.375 89.60625) (end 147.4125 89.64375) (width 0.2) (layer "F.Cu") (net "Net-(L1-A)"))
 (segment (start 147.375 87.89375) (end 147.375 89.60625) (width 0.2) (layer "F.Cu") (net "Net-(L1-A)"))
 (segment (start 145.375 103.58) (end 145.7925 103.58) (width 0.2) (layer "F.Cu") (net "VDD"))
 (segment (start 144.375 93.25) (end 142.625 95) (width 0.2) (layer "F.Cu") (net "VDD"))
 (segment (start 144.375 93.25) (end 147.125 93.25) (width 0.2) (layer "F.Cu") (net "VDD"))
 (segment (start 142.625 95) (end 142.625 103.25) (width 0.2) (layer "F.Cu") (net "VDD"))
 (segment (start 152.625 93) (end 152.625 92.2125) (width 0.2) (layer "F.Cu") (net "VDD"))
 (segment (start 152.6375 92.2) (end 152.6375 90.45) (width 0.2) (layer "F.Cu") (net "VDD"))
 (segment (start 142.625 103.25) (end 142.955 103.58) (width 0.2) (layer "F.Cu") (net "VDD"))
 (segment (start 144.375 93.25) (end 145.5875 92.0375) (width 0.2) (layer "F.Cu") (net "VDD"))
 (segment (start 152.375 93.25) (end 152.625 93) (width 0.2) (layer "F.Cu") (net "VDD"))
 (segment (start 148.875 93.25) (end 152.375 93.25) (width 0.2) (layer "F.Cu") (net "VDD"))
 (segment (start 142.955 103.58) (end 145.375 103.58) (width 0.2) (layer "F.Cu") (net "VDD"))
 (segment (start 145.5875 92.0375) (end 145.5875 89.64375) (width 0.2) (layer "F.Cu") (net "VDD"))
 (segment (start 152.625 92.2125) (end 152.6375 92.2) (width 0.2) (layer "F.Cu") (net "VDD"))
 (segment (start 154.925 89.35) (end 153.625 89.35) (width 0.2) (layer "F.Cu") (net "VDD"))
 (segment (start 150.55 108.3375) (end 156.875 108.3375) (width 0.2) (layer "F.Cu") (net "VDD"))
 (segment (start 145.7925 103.58) (end 150.55 108.3375) (width 0.2) (layer "F.Cu") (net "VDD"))
 (segment (start 153.625 89.35) (end 152.6375 90.3375) (width 0.2) (layer "F.Cu") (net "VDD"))
 (via (at 147.125 93.25) (size 0.6) (drill 0.3) (layers "F.Cu" "B.Cu") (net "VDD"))
 (via (at 148.875 93.25) (size 0.6) (drill 0.3) (layers "F.Cu" "B.Cu") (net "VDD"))
 (segment (start 148.875 93.25) (end 147.125 93.25) (width 0.2) (layer "B.Cu") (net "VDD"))
 (segment (start 154.025 90.2) (end 154.475 89.75) (width 0.2) (layer "F.Cu") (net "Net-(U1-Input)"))
 (segment (start 154.475 89.75) (end 154.925 89.75) (width 0.2) (layer "F.Cu") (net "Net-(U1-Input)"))
 (segment (start 154.025 92.1325) (end 154.025 90.2) (width 0.2) (layer "F.Cu") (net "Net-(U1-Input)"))
 (segment (start 154.1128 102.6422) (end 153.0746 103.6804) (width 0.2) (layer "F.Cu") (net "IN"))
 (segment (start 154.025 93.2675) (end 154.1128 93.3553) (width 0.2) (layer "F.Cu") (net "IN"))
 (segment (start 152.1675 104.5875) (end 153.0746 103.6804) (width 0.2) (layer "F.Cu") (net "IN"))
 (segment (start 154.1128 93.3553) (end 154.1128 102.6422) (width 0.2) (layer "F.Cu") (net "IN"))
 (segment (start 149.125 104.5875) (end 152.1675 104.5875) (width 0.2) (layer "F.Cu") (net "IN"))
 (segment (start 157.125 110.4125) (end 153.5025 110.4125) (width 0.2) (layer "F.Cu") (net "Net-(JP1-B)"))
 (segment (start 153.5025 110.4125) (end 153.415 110.5) (width 0.2) (layer "F.Cu") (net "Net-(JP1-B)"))
 (segment (start 154.925 106.7) (end 154.925 90.15) (width 0.2) (layer "F.Cu") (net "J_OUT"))
 (segment (start 154.125 107.5) (end 154.925 106.7) (width 0.2) (layer "F.Cu") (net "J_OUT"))
 (via (at 154.125 107.5) (size 0.6) (drill 0.3) (layers "F.Cu" "B.Cu") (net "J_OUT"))
 (segment (start 151.125 110.5) (end 150.875 110.5) (width 0.2) (layer "B.Cu") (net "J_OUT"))
 (segment (start 154.125 107.5) (end 151.125 110.5) (width 0.2) (layer "B.Cu") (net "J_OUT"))
 (segment (start 155.325 90.15) (end 156.525 91.35) (width 0.2) (layer "F.Cu") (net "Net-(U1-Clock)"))
 (segment (start 156.525 91.35) (end 156.525 92.1025) (width 0.2) (layer "F.Cu") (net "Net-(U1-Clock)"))
 (segment (start 155.125 87.5) (end 155.625 88) (width 0.2) (layer "F.Cu") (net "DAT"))
 (segment (start 147.875 96.25) (end 147.875 91.5) (width 0.2) (layer "F.Cu") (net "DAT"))
 (segment (start 145.625 98.5) (end 147.875 96.25) (width 0.2) (layer "F.Cu") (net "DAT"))
 (segment (start 147.875 91.5) (end 151.875 87.5) (width 0.2) (layer "F.Cu") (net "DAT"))
 (segment (start 155.625 89.05) (end 155.325 89.35) (width 0.2) (layer "F.Cu") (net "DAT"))
 (segment (start 151.875 87.5) (end 155.125 87.5) (width 0.2) (layer "F.Cu") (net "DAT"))
 (segment (start 145.375 98.5) (end 145.625 98.5) (width 0.2) (layer "F.Cu") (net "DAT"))
 (segment (start 155.625 88) (end 155.625 89.05) (width 0.2) (layer "F.Cu") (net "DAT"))
 (segment (start 147.835 101.04) (end 151.25 97.625) (width 0.2) (layer "F.Cu") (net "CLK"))
 (segment (start 145.375 101.04) (end 147.835 101.04) (width 0.2) (layer "F.Cu") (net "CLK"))
 (via (at 151.25 97.625) (size 0.6) (drill 0.3) (layers "F.Cu" "B.Cu") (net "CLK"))
 (via (at 156.525 93.2975) (size 0.6) (drill 0.3) (layers "F.Cu" "B.Cu") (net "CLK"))
 (segment (start 155.5775 93.2975) (end 156.525 93.2975) (width 0.2) (layer "B.Cu") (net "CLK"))
 (segment (start 151.25 97.625) (end 155.5775 93.2975) (width 0.2) (layer "B.Cu") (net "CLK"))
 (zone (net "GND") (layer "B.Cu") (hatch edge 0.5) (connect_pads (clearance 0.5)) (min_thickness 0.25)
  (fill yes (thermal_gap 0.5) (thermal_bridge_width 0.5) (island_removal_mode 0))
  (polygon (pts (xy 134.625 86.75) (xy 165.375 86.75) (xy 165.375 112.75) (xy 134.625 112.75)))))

